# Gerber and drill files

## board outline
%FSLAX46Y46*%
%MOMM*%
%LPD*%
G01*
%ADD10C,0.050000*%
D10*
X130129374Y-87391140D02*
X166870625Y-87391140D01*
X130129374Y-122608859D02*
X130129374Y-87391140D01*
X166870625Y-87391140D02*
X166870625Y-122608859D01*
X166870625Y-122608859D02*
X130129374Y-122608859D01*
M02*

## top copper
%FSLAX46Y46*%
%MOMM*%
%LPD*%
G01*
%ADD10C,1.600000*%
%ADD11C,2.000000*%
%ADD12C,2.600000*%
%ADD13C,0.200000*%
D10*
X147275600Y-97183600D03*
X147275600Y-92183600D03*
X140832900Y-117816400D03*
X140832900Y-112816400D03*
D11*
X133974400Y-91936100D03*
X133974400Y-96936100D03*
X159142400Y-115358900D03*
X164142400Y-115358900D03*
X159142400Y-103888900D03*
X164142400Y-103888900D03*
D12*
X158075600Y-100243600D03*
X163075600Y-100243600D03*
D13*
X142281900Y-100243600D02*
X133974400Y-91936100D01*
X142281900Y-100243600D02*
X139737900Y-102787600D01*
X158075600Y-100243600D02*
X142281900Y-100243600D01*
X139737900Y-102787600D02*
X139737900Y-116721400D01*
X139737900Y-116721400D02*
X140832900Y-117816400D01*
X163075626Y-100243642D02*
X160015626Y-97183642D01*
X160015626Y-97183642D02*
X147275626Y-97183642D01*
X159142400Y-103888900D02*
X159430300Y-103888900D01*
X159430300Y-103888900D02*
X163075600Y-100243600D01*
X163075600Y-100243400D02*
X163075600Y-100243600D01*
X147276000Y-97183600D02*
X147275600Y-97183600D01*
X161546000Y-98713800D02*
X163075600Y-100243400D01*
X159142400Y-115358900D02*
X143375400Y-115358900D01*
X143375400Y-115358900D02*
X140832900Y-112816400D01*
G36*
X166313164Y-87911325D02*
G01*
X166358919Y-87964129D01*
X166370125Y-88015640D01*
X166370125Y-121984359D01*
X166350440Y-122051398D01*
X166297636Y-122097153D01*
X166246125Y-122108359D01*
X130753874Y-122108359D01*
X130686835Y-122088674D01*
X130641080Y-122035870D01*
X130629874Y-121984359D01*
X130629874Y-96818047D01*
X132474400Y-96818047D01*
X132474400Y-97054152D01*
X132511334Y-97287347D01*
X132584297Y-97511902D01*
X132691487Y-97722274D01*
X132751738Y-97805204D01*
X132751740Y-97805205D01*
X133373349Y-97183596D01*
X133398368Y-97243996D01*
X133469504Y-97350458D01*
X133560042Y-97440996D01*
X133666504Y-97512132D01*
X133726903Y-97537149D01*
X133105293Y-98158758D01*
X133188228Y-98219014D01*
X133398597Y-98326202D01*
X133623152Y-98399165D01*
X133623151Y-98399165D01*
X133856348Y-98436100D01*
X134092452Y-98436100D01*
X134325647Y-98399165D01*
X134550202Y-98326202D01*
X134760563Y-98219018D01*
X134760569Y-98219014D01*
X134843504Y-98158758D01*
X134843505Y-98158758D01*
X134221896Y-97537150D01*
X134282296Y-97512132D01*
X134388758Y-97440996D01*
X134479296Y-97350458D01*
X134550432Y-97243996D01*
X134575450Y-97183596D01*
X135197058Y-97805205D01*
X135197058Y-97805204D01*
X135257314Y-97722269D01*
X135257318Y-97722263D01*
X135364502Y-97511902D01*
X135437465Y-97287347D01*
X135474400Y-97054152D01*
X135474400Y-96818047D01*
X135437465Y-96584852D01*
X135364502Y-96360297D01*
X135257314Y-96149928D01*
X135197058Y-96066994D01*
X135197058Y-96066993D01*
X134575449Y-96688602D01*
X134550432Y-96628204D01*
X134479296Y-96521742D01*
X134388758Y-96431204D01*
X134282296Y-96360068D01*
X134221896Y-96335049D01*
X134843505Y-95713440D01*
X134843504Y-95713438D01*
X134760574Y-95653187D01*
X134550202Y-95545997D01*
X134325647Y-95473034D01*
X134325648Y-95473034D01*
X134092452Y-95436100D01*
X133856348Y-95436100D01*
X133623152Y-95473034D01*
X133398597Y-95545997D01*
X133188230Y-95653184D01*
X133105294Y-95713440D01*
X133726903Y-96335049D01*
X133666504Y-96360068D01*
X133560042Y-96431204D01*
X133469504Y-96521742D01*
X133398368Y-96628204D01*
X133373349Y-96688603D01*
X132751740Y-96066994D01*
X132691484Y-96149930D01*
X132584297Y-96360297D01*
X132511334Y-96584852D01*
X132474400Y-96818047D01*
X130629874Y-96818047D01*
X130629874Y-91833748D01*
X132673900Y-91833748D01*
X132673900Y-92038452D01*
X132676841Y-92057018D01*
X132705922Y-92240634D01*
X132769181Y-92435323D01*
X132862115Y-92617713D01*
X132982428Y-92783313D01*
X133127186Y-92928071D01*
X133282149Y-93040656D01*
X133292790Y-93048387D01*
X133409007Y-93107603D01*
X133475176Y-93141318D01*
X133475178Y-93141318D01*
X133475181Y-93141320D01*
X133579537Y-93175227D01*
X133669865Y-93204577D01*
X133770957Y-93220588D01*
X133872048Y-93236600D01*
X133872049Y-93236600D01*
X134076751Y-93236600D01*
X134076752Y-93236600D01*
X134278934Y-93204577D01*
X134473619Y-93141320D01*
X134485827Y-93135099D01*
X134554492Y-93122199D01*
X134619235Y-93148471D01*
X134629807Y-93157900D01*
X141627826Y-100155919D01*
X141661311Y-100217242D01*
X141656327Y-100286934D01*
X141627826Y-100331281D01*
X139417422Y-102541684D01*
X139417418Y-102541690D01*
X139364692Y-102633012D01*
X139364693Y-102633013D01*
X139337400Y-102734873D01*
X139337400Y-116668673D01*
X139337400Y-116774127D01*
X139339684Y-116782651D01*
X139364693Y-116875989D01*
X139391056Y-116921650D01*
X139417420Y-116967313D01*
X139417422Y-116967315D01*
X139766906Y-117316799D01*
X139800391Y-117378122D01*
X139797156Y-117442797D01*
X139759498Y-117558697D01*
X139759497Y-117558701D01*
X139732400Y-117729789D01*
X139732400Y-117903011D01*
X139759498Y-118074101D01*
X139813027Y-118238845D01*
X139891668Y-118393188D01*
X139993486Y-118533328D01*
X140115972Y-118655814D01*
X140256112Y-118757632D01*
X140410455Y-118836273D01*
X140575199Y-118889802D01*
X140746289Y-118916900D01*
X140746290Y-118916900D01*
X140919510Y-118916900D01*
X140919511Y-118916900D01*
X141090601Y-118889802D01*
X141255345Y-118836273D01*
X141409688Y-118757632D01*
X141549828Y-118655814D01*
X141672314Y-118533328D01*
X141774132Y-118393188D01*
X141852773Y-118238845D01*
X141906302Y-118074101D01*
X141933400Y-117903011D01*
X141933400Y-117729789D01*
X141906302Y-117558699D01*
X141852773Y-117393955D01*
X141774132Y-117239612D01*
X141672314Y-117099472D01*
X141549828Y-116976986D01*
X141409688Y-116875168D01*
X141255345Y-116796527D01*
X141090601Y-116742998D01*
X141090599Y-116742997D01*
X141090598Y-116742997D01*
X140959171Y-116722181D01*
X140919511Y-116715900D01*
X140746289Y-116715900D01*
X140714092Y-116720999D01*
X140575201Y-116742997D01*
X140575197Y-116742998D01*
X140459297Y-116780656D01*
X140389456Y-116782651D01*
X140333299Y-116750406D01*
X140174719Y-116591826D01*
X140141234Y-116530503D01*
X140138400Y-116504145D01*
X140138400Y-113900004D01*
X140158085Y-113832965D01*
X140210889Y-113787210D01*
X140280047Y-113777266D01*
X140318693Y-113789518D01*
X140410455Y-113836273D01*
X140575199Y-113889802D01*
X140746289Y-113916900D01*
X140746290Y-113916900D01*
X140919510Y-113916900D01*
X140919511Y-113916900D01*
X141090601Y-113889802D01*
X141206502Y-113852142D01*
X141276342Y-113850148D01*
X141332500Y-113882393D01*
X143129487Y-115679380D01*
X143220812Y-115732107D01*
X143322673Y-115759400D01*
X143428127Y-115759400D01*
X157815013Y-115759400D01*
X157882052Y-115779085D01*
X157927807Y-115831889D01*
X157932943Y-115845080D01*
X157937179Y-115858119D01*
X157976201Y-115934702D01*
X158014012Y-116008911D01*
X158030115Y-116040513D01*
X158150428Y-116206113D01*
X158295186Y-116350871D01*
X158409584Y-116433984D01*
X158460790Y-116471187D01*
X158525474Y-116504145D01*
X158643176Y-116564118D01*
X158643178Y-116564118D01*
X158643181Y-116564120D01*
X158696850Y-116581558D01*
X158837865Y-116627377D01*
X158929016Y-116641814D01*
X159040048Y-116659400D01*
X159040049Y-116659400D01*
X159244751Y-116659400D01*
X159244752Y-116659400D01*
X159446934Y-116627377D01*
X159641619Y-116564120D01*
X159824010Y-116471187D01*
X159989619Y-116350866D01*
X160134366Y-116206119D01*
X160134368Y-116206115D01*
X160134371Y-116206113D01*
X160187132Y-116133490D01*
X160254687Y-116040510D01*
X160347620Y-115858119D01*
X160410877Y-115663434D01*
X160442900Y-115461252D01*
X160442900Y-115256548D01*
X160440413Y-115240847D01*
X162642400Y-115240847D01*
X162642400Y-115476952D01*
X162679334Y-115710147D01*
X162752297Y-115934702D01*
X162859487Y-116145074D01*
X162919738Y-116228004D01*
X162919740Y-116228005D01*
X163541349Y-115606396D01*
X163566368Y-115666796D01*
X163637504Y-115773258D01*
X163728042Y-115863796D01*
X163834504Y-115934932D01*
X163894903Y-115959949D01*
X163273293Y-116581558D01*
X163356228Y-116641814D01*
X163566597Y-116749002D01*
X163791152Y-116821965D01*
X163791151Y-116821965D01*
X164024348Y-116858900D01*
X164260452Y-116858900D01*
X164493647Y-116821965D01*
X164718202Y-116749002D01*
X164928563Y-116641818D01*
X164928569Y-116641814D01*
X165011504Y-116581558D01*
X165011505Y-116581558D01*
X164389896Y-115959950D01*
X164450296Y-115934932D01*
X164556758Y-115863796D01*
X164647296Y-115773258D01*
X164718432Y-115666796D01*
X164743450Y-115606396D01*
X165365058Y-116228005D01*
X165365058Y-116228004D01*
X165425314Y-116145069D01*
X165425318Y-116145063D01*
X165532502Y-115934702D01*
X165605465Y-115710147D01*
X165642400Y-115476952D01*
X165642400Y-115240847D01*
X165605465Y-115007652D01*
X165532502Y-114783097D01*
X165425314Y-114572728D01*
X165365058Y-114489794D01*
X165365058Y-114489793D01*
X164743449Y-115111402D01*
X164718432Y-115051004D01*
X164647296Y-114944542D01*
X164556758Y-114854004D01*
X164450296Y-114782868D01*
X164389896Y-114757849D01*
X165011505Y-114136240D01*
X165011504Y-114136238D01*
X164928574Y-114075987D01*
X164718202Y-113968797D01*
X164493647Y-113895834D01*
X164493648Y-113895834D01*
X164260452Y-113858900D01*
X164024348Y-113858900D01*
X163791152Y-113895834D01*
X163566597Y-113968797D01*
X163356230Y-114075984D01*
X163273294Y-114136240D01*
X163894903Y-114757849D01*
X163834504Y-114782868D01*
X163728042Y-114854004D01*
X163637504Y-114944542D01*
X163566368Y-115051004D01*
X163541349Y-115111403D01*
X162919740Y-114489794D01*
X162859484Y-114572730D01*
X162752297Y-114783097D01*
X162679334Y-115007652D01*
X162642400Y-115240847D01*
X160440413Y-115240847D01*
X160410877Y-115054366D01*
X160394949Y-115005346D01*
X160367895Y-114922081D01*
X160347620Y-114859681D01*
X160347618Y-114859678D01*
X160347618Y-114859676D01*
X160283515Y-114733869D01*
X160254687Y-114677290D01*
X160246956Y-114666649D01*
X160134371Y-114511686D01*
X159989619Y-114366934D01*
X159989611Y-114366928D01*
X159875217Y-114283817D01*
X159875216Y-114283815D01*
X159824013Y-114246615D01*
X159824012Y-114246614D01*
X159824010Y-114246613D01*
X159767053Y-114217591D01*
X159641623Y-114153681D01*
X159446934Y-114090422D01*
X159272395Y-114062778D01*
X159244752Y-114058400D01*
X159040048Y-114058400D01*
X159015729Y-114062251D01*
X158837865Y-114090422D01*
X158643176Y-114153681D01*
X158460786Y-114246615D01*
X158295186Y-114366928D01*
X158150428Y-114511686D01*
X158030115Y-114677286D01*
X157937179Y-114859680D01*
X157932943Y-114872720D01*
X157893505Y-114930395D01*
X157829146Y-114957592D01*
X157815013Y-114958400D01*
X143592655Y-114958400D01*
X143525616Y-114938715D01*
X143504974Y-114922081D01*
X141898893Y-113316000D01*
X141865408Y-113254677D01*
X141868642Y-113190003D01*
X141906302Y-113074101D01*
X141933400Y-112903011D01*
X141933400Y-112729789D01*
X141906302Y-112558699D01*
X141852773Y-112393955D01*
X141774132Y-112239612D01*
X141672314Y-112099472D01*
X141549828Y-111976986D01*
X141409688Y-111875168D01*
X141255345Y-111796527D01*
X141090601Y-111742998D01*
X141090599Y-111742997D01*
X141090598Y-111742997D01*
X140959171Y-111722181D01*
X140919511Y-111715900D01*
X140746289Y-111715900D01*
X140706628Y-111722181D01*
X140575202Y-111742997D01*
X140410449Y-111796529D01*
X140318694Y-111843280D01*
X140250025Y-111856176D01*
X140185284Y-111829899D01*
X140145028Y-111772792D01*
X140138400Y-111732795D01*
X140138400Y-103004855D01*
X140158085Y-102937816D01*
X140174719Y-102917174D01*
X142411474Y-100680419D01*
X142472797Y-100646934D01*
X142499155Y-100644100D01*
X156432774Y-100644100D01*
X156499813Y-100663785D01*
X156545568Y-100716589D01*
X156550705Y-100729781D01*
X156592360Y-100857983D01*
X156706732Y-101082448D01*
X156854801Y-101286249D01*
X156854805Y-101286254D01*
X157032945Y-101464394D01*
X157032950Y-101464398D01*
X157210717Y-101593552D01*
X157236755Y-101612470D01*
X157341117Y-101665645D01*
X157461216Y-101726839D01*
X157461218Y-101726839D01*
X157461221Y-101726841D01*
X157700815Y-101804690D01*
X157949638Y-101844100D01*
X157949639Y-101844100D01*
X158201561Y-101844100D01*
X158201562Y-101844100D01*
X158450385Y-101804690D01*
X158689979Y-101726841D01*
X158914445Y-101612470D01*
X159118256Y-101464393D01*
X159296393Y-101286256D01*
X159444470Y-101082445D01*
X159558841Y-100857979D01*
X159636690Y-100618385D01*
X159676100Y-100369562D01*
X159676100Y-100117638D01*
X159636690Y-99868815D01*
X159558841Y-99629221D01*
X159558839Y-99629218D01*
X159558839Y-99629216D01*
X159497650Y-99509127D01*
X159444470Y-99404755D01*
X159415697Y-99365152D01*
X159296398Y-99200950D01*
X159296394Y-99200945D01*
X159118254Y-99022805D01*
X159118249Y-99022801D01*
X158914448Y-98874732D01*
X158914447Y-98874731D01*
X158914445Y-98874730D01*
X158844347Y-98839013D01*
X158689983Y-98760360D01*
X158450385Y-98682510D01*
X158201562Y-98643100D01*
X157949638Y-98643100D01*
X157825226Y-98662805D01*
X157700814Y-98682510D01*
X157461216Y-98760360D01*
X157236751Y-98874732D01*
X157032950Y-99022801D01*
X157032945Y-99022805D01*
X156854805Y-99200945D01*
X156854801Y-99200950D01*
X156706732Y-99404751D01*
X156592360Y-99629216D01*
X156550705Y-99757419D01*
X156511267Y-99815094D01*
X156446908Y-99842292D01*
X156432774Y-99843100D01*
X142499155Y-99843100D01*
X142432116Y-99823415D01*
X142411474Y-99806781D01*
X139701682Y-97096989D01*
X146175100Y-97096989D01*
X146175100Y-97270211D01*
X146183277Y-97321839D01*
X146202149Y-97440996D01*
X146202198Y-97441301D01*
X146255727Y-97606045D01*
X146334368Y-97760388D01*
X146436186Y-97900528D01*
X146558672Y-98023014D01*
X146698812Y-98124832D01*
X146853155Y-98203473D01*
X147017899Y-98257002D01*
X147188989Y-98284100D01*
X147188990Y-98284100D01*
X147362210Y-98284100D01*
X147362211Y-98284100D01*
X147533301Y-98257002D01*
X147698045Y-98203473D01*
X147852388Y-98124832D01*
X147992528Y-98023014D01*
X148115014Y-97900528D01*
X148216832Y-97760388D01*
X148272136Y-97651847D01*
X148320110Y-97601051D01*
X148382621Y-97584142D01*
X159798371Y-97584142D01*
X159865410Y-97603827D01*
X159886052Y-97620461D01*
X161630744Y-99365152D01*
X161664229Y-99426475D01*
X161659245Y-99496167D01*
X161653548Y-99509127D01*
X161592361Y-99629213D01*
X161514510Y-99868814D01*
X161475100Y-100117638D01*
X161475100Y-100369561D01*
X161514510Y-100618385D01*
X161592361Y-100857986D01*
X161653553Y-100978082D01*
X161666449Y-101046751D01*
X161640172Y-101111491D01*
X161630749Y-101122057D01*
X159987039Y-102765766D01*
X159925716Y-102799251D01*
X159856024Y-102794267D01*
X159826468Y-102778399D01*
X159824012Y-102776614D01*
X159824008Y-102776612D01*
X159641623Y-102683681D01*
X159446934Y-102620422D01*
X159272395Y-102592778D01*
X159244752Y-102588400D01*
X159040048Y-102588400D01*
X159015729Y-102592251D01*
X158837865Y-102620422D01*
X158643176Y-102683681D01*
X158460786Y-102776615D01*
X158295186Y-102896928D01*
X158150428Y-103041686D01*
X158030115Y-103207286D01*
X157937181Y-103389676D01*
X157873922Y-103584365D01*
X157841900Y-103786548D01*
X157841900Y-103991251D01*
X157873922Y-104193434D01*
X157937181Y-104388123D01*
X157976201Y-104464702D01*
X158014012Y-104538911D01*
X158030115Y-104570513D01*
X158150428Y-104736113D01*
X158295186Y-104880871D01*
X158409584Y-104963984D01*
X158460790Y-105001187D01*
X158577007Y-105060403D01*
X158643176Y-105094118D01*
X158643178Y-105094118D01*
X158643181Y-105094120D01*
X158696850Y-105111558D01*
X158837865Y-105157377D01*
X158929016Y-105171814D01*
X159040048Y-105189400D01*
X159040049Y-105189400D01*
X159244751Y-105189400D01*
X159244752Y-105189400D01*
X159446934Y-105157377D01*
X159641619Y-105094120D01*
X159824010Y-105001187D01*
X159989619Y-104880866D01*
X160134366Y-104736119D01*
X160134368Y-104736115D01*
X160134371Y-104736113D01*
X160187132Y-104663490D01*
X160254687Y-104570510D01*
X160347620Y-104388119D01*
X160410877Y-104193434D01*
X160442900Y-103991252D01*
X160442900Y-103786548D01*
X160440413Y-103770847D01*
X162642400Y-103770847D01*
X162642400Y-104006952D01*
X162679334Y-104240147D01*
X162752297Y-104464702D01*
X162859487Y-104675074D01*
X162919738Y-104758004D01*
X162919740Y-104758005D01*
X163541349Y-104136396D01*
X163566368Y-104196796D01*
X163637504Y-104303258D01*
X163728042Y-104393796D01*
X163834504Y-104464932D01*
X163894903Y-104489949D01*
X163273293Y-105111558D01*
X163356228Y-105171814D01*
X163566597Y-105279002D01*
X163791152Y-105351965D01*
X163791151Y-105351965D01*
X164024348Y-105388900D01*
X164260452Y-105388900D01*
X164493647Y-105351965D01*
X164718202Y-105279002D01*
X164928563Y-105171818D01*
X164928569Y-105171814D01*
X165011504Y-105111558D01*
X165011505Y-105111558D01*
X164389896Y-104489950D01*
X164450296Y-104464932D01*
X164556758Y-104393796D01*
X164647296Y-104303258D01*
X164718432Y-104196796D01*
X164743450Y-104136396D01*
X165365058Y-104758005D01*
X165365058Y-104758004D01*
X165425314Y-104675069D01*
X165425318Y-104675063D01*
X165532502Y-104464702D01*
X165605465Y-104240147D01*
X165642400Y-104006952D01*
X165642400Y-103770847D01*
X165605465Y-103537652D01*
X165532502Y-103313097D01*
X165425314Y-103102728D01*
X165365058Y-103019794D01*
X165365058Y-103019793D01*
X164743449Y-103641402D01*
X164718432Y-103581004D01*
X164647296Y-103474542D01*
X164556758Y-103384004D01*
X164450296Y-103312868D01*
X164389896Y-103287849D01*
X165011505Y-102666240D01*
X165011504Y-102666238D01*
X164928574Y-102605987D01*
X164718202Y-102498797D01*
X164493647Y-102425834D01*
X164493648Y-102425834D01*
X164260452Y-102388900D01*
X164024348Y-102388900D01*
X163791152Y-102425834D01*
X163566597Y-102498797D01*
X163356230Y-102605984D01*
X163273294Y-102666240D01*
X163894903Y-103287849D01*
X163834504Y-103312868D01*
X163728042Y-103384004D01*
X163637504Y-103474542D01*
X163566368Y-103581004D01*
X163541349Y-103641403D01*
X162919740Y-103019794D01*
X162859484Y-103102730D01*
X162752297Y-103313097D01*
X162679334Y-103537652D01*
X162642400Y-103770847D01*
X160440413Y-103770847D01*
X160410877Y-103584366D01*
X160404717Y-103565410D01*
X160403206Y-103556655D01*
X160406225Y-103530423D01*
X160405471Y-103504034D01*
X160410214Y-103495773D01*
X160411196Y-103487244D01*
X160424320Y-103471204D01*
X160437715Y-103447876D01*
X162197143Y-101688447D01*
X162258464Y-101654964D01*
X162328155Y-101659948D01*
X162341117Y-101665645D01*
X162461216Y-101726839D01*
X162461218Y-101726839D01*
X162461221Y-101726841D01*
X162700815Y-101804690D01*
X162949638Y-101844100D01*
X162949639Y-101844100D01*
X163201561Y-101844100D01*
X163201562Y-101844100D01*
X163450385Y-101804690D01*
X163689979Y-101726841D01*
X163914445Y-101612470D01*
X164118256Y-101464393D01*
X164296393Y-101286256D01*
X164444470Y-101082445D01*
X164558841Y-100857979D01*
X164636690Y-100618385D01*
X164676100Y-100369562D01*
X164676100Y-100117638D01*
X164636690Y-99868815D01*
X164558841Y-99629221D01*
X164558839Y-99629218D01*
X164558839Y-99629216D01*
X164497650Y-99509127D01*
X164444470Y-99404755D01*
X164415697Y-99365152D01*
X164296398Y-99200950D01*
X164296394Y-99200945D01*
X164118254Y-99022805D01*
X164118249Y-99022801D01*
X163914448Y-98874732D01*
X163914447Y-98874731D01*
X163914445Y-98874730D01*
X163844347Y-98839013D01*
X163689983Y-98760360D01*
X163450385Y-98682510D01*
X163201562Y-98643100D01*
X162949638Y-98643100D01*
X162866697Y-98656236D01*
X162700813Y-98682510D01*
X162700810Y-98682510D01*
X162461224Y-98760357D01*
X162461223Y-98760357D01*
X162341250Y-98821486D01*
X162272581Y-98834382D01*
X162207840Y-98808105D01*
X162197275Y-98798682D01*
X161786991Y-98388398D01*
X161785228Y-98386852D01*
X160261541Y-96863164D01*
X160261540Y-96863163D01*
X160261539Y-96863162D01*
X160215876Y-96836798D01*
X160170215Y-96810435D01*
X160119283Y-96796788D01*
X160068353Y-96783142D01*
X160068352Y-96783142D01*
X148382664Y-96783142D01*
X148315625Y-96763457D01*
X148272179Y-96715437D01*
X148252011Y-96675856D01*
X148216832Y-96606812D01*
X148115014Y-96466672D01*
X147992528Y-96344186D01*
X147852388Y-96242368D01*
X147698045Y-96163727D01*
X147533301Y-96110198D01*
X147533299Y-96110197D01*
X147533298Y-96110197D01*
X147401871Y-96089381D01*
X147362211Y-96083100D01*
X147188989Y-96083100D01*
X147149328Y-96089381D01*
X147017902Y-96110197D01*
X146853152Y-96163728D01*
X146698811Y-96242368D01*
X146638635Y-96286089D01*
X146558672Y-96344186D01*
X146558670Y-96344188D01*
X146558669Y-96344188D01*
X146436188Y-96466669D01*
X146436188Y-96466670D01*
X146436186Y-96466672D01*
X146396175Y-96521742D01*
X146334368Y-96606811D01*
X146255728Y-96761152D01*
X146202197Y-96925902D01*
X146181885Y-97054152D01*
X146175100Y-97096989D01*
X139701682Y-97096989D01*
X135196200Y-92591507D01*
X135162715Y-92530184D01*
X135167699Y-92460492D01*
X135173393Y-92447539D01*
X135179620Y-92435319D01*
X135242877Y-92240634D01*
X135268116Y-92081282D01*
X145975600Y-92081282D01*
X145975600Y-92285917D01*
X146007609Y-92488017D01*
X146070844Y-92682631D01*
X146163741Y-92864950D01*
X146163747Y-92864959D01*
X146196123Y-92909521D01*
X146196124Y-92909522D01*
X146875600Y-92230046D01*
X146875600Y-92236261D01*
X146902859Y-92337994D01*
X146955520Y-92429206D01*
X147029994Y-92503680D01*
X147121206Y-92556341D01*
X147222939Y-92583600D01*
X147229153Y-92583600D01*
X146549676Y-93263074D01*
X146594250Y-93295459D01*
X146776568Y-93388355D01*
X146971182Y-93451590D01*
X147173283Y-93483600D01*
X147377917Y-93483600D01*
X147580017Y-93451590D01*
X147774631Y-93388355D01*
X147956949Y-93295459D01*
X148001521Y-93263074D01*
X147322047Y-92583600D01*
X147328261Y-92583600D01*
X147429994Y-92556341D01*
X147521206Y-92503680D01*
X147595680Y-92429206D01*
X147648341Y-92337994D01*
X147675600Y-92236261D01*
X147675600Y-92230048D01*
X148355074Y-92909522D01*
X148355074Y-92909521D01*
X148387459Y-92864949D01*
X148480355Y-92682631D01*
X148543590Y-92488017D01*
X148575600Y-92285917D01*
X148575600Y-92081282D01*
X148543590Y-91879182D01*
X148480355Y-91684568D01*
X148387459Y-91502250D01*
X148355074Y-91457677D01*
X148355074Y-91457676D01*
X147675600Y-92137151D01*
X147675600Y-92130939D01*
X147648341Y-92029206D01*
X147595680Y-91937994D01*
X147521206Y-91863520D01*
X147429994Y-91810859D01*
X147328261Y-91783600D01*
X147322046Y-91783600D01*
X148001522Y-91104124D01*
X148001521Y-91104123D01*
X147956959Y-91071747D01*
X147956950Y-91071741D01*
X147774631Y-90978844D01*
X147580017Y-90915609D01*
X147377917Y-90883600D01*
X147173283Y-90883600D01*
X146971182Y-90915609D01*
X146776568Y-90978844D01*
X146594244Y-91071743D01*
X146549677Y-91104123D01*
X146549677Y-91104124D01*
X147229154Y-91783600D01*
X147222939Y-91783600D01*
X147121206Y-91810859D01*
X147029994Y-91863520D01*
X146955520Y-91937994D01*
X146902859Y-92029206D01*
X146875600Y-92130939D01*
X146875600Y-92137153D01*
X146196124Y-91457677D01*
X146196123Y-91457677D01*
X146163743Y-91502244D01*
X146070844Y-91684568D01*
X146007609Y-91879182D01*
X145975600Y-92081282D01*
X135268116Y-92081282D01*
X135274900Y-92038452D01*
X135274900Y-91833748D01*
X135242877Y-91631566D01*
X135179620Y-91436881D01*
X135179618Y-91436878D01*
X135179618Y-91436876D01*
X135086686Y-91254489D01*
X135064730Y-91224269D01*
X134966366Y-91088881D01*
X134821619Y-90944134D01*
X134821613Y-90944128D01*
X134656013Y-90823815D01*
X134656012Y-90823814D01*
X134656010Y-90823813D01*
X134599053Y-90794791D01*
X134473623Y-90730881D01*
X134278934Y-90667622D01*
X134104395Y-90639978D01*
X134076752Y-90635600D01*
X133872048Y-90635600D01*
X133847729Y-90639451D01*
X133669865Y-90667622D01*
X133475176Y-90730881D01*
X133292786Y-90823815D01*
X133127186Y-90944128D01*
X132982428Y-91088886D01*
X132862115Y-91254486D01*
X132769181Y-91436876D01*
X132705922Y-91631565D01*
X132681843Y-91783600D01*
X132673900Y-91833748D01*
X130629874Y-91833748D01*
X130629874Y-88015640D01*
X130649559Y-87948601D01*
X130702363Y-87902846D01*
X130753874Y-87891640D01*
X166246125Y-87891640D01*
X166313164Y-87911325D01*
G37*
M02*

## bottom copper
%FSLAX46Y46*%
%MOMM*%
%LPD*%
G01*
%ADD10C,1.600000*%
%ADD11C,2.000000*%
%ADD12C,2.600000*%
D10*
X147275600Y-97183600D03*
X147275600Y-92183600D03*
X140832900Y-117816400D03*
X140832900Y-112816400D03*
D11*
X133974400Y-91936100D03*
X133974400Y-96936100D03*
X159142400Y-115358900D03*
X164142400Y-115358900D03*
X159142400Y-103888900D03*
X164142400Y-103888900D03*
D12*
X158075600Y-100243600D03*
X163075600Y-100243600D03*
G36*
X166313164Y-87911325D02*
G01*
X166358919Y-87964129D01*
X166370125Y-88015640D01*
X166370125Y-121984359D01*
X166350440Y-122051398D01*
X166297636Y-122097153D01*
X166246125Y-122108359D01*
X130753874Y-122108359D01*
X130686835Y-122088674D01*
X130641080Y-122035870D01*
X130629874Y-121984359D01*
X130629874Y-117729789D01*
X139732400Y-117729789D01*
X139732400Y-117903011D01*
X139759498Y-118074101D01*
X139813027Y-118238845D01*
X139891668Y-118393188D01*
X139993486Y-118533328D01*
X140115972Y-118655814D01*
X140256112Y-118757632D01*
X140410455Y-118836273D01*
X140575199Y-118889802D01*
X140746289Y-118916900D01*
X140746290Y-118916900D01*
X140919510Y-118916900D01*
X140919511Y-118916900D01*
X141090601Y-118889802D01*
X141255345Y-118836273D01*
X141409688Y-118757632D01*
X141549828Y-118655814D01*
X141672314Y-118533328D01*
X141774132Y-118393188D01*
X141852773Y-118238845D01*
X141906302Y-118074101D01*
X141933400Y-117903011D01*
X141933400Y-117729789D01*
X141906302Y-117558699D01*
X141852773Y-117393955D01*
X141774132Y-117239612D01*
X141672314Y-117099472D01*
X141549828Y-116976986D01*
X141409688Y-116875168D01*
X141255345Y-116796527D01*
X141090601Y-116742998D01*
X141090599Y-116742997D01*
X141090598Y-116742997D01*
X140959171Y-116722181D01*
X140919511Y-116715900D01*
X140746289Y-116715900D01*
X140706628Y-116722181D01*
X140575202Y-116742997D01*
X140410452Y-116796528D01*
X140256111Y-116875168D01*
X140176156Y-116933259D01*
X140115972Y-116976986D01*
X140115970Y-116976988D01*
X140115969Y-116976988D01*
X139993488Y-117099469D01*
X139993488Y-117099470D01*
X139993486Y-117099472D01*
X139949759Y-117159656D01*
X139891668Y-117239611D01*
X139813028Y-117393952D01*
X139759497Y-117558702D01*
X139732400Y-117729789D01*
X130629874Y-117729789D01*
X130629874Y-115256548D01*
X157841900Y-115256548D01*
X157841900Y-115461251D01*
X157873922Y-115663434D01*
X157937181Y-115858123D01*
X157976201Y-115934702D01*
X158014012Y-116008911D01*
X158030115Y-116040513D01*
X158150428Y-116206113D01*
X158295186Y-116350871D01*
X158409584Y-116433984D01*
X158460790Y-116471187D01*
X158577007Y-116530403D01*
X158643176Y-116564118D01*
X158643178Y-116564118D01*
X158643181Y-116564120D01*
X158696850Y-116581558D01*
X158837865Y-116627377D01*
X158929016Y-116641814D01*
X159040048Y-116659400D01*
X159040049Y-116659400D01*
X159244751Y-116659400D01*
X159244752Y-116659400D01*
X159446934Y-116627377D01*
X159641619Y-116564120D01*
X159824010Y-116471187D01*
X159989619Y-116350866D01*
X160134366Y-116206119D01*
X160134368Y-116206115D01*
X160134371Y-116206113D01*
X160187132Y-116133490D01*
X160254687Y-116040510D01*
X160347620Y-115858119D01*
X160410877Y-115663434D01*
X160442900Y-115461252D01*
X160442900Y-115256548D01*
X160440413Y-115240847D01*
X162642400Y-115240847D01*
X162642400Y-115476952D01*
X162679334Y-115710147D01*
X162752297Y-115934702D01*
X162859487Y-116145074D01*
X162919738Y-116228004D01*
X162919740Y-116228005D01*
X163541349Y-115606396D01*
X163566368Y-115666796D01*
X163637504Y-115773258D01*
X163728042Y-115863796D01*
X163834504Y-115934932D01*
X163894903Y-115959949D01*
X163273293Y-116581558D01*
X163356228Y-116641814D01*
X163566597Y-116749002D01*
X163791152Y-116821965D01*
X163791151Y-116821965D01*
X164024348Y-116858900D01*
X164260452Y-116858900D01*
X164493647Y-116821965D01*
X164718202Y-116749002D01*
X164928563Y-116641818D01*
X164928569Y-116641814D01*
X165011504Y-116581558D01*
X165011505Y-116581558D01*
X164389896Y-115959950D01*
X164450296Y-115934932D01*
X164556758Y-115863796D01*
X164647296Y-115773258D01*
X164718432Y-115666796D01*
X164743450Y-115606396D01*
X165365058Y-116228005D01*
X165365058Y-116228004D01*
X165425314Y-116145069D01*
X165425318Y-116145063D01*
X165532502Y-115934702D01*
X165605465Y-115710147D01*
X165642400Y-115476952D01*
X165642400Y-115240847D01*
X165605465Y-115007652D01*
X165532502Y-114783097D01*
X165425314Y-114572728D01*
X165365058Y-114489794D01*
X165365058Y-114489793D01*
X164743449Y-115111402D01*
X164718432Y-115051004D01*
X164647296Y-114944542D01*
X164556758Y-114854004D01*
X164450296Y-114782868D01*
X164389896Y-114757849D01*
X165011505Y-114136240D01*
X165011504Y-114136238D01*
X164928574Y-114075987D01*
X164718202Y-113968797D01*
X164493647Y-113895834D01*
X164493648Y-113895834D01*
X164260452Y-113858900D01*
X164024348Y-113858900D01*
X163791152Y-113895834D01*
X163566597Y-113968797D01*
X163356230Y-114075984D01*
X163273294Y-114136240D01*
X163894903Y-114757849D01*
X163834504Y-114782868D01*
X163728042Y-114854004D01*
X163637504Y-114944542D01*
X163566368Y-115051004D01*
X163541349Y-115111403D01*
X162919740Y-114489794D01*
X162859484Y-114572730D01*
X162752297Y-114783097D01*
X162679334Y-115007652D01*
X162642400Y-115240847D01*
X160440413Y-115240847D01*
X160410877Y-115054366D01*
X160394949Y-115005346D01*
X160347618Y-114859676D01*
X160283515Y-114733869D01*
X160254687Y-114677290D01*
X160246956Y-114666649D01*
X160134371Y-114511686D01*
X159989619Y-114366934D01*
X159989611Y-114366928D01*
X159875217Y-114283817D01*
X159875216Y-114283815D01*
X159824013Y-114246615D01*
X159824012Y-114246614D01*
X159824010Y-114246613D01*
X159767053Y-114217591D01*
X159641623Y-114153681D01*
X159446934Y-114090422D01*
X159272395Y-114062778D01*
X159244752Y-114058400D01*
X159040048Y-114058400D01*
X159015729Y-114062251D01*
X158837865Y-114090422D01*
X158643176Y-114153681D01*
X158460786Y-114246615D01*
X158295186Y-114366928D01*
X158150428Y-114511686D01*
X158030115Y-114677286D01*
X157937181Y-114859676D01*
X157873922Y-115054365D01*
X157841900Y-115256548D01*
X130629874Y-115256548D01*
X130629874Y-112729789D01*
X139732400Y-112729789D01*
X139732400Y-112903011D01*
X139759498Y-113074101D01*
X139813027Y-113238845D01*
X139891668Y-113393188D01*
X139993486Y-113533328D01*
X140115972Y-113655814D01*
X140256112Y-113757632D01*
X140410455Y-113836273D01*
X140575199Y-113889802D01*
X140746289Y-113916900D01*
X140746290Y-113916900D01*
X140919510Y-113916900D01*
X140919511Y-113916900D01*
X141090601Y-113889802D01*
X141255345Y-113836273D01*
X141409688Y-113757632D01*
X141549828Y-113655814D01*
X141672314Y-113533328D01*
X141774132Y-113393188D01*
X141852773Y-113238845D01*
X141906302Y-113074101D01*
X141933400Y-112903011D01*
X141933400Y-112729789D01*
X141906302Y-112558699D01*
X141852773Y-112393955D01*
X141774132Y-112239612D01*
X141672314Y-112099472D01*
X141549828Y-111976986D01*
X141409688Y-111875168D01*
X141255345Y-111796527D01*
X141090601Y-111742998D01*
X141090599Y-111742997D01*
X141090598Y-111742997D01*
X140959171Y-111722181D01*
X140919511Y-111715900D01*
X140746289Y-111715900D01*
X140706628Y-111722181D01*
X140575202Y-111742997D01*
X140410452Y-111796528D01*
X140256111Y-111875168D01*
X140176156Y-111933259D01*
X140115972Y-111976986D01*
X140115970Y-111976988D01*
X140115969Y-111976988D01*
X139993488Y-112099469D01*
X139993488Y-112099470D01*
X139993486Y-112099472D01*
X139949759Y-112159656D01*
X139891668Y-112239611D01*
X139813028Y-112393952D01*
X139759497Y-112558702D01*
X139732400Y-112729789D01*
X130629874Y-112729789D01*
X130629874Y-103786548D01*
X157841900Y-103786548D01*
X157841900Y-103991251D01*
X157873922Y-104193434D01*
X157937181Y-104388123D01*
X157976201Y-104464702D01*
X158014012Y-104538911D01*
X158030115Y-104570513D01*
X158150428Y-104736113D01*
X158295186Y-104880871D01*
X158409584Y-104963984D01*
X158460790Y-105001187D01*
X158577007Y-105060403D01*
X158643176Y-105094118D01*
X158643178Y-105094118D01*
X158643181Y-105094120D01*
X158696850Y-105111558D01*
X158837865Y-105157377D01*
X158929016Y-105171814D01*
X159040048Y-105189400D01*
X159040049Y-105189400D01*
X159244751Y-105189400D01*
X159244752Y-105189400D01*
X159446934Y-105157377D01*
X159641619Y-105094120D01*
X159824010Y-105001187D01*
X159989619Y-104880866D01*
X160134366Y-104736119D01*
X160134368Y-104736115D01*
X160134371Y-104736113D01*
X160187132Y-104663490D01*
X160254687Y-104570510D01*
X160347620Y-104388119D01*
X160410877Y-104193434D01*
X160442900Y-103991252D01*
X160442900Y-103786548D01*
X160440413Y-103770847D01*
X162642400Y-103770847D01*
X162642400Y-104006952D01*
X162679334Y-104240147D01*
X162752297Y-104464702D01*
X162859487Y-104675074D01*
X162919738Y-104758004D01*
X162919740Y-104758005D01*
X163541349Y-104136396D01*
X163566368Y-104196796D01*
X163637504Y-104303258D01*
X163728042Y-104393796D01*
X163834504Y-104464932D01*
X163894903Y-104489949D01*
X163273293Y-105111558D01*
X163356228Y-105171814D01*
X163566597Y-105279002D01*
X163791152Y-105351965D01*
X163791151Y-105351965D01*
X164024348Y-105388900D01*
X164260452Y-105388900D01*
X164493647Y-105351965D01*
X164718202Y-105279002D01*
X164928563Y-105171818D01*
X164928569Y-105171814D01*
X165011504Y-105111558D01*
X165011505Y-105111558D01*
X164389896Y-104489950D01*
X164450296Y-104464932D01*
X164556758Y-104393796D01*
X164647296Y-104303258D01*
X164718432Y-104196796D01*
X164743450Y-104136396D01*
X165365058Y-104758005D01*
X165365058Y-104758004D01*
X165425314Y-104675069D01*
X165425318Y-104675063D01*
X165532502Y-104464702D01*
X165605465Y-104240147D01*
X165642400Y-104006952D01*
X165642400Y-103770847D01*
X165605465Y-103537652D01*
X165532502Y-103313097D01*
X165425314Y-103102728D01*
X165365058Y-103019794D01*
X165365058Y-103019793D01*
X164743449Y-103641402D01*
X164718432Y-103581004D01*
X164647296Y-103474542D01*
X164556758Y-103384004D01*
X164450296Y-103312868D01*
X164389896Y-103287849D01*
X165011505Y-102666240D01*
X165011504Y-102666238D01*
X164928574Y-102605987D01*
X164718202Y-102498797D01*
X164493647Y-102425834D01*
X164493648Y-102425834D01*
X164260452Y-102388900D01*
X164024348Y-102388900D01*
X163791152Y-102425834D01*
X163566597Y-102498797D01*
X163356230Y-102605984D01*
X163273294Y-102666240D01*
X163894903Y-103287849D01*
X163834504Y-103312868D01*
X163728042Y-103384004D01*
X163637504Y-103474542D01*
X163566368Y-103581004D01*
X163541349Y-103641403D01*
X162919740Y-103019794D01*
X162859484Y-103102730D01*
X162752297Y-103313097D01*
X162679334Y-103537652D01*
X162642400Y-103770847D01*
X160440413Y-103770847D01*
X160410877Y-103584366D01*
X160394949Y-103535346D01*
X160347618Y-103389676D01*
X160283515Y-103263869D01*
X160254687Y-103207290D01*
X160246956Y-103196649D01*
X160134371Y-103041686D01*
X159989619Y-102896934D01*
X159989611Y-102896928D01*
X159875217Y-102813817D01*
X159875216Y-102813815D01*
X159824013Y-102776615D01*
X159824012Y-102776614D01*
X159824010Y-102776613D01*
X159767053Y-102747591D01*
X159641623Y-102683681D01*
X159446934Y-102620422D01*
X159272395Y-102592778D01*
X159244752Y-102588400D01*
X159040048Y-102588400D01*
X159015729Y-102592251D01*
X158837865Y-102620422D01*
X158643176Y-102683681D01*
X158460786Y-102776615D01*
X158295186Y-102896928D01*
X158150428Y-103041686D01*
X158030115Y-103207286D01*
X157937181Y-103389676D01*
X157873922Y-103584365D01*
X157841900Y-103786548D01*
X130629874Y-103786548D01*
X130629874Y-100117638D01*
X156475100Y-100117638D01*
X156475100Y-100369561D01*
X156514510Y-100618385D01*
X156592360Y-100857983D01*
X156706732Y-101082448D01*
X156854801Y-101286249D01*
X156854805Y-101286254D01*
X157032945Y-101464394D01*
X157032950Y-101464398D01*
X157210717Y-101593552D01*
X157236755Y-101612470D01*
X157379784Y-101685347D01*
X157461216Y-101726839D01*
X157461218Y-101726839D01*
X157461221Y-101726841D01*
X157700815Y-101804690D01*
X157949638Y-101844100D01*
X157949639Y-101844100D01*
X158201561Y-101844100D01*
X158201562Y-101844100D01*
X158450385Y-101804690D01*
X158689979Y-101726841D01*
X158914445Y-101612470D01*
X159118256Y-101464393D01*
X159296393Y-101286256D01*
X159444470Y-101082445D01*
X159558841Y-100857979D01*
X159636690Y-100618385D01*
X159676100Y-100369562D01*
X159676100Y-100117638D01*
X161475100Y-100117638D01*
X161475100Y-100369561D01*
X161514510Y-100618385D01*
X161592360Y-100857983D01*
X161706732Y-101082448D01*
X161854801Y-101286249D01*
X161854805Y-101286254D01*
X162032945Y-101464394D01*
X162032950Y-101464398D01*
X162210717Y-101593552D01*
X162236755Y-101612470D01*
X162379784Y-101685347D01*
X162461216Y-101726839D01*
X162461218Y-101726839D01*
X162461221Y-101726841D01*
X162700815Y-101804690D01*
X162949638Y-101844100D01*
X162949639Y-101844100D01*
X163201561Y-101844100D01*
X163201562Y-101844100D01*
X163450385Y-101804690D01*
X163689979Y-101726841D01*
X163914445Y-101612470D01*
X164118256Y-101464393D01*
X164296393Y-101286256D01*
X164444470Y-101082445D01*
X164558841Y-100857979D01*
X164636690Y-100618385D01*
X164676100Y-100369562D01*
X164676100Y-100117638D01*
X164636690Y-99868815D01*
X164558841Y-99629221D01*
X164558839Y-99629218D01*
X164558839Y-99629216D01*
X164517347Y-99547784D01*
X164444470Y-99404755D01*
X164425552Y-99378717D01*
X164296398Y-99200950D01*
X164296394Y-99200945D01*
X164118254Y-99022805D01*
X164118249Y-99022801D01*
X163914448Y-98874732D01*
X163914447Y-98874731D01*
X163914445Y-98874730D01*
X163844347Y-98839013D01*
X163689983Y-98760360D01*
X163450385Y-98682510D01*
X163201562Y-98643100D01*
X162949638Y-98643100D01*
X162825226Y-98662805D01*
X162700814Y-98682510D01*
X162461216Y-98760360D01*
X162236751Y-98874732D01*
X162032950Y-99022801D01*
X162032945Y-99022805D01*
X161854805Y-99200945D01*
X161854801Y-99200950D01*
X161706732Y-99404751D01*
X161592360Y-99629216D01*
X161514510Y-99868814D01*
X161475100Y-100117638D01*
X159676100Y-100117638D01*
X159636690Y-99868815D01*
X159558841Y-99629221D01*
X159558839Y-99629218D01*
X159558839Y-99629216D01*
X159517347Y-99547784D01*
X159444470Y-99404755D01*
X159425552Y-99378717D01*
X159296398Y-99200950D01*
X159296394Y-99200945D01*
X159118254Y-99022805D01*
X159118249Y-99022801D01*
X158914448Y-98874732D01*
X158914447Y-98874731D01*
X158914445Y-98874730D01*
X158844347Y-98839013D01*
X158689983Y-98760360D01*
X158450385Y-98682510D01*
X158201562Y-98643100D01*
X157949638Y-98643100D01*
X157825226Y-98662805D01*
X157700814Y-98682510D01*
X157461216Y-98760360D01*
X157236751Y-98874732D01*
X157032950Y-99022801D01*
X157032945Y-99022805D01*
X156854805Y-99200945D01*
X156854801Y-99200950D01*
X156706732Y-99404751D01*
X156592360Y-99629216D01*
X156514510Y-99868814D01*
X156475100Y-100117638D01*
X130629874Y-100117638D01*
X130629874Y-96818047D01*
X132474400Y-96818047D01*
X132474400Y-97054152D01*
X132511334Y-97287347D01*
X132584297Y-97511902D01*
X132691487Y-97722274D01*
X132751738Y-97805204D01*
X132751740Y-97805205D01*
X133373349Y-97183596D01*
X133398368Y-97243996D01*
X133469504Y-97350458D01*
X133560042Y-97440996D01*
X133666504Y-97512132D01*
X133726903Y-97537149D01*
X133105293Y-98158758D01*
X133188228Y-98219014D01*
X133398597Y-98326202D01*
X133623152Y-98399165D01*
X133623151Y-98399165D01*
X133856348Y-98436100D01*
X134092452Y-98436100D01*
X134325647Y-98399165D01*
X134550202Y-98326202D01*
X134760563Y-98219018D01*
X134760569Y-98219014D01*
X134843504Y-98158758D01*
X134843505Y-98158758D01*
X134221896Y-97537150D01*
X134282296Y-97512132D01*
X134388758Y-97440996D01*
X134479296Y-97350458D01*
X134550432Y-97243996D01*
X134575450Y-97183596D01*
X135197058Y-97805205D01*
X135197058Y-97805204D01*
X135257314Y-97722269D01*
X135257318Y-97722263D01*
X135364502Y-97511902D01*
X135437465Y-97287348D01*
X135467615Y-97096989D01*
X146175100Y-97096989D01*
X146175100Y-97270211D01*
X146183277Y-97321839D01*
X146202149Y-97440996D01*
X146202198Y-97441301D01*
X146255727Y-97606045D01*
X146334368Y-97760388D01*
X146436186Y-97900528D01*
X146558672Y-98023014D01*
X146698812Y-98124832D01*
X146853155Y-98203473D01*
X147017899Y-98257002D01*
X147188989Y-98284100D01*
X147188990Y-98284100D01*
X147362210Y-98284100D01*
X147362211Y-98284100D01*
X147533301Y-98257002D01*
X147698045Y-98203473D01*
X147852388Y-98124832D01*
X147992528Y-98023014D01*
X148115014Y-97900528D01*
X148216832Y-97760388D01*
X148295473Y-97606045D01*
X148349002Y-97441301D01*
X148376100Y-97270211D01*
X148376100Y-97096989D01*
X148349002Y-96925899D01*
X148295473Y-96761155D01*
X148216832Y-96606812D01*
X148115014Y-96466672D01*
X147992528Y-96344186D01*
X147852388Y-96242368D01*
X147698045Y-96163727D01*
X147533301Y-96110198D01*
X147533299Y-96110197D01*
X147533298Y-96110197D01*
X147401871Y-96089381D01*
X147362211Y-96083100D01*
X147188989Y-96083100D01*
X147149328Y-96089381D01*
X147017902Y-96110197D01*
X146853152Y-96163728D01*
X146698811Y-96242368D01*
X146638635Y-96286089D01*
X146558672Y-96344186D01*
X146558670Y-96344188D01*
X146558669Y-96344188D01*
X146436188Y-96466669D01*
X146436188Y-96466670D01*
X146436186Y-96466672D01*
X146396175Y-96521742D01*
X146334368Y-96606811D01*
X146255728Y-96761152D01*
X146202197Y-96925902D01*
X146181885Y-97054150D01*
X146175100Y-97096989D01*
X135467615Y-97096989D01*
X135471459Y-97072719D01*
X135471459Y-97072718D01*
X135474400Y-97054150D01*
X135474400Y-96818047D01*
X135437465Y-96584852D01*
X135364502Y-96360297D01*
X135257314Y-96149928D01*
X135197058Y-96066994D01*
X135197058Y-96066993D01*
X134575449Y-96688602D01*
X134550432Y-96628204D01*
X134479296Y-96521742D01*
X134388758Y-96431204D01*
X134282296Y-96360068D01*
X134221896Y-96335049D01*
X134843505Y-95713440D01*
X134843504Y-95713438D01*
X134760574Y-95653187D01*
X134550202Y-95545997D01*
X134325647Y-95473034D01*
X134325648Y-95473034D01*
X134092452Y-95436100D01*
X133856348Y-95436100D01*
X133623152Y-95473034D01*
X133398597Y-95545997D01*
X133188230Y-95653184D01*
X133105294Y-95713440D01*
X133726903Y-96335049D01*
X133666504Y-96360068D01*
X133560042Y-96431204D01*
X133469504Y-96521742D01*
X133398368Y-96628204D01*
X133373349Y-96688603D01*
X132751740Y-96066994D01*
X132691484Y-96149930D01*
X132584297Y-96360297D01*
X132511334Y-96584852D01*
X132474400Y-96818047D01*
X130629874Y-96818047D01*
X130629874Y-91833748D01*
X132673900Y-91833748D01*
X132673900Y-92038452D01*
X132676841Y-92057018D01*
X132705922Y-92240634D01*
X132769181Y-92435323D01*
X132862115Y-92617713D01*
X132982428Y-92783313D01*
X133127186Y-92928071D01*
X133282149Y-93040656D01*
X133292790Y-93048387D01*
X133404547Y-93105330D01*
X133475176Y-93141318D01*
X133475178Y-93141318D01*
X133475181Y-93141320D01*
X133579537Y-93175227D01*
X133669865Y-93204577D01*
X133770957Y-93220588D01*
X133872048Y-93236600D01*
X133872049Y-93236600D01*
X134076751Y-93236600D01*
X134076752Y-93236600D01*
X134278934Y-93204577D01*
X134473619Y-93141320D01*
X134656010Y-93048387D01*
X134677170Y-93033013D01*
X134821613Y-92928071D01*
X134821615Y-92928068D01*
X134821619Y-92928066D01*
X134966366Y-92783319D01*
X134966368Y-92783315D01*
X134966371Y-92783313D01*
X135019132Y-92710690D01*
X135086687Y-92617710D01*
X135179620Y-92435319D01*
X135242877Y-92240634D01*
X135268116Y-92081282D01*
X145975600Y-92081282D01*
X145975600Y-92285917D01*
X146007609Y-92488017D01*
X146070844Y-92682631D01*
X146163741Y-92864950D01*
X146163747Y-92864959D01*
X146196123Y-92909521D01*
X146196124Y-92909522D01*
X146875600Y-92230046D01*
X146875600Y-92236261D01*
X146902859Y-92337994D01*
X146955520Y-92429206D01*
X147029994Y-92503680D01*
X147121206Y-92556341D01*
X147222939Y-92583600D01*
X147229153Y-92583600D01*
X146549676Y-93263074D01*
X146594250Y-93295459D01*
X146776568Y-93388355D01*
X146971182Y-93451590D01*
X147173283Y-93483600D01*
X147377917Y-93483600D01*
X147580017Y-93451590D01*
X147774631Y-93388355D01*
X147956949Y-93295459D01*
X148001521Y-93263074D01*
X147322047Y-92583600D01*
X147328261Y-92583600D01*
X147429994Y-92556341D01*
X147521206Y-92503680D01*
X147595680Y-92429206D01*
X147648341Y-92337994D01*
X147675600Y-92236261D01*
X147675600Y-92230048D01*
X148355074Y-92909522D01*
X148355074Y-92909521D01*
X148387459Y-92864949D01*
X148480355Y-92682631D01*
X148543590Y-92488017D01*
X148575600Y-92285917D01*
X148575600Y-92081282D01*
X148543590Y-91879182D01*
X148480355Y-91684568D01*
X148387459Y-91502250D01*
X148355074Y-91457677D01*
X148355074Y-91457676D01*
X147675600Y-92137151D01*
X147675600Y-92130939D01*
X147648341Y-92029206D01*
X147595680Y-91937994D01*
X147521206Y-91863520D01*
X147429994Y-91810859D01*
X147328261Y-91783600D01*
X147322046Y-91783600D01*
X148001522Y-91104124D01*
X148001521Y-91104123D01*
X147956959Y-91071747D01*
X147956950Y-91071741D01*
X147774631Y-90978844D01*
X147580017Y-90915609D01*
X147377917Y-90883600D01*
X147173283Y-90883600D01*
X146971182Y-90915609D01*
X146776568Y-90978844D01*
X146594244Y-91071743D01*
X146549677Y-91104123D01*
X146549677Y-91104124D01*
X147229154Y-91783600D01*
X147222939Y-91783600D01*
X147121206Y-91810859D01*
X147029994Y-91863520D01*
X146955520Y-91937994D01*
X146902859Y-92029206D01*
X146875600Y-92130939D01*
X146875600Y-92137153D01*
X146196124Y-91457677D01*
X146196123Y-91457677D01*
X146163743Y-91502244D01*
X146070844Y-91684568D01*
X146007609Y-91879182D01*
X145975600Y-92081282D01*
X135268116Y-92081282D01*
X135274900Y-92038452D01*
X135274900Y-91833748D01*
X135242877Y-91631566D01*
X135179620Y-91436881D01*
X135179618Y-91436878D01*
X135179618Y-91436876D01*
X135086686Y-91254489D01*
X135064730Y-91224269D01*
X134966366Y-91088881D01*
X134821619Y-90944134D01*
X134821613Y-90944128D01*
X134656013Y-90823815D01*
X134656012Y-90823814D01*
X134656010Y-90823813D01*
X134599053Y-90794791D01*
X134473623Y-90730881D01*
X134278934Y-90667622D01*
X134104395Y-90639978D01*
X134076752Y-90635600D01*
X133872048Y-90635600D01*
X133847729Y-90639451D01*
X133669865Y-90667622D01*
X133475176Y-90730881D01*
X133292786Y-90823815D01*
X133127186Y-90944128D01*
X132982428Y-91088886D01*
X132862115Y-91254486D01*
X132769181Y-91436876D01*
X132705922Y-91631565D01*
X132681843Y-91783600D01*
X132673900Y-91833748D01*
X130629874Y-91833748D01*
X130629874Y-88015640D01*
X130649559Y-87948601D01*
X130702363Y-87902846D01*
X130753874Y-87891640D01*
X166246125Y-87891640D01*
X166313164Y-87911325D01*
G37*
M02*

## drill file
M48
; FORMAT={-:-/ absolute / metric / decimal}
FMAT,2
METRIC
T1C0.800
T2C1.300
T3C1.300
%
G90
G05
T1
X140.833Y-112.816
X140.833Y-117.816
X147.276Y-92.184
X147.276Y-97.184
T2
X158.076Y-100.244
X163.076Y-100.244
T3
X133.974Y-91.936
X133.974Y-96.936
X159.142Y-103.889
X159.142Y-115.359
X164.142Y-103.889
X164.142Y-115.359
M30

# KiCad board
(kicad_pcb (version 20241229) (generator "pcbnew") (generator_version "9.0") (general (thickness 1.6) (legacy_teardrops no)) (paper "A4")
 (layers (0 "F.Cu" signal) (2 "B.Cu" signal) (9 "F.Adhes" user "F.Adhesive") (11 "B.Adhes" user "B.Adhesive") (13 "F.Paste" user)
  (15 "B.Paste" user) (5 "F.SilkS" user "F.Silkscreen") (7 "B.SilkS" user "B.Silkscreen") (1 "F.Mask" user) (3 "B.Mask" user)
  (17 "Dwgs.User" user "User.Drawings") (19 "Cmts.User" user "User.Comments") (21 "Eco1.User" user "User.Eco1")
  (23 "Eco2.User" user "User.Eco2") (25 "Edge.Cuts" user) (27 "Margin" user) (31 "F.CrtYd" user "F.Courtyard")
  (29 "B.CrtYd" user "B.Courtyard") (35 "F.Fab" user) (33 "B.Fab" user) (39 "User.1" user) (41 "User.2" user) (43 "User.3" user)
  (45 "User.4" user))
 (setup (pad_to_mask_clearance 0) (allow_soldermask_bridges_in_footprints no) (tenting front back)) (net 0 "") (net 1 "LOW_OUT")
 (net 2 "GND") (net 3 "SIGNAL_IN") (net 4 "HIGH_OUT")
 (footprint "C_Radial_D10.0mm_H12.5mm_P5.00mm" (layer "F.Cu") (at 147.2756 97.1836 90)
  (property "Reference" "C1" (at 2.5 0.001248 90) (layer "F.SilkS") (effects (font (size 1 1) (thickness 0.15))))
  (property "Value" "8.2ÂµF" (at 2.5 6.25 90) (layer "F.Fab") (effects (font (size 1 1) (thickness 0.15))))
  (pad "1" thru_hole circle (at 0 0 90) (size 1.6 1.6) (drill 0.8) (layers "*.Cu" "*.Mask") (remove_unused_layers no) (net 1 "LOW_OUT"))
  (pad "2" thru_hole circle (at 5 0 90) (size 1.6 1.6) (drill 0.8) (layers "*.Cu" "*.Mask") (remove_unused_layers no) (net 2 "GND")))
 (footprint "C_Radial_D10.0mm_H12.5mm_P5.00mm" (layer "F.Cu") (at 140.8329 117.8164 90)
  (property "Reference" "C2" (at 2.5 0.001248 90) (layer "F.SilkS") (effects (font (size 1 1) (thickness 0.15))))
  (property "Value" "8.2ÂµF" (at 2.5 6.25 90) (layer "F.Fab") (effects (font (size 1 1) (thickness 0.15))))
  (pad "1" thru_hole circle (at 0 0 90) (size 1.6 1.6) (drill 0.8) (layers "*.Cu" "*.Mask") (remove_unused_layers no) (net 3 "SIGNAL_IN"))
  (pad "2" thru_hole circle (at 5 0 90) (size 1.6 1.6) (drill 0.8) (layers "*.Cu" "*.Mask") (remove_unused_layers no) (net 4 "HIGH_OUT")))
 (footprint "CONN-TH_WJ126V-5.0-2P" (layer "F.Cu") (at 133.9744 94.4361)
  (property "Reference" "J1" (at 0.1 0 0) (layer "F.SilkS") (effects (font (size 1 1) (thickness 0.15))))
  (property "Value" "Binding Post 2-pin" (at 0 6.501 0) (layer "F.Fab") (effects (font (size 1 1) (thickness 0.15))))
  (pad "1" thru_hole circle (at 0 -2.5) (size 2 2) (drill 1.300022) (layers "*.Cu" "*.Mask") (remove_unused_layers no) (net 3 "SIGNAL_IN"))
  (pad "2" thru_hole circle (at 0 2.5) (size 2 2) (drill 1.300022) (layers "*.Cu" "*.Mask") (remove_unused_layers no) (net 2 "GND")))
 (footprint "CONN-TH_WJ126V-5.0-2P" (layer "F.Cu") (at 161.6424 115.3589 90)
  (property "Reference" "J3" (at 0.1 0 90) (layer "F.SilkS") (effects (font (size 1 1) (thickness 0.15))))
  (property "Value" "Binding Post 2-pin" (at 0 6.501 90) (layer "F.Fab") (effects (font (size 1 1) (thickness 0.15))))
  (pad "1" thru_hole circle (at 0 -2.5 90) (size 2 2) (drill 1.300022) (layers "*.Cu" "*.Mask") (remove_unused_layers no) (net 4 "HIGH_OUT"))
  (pad "2" thru_hole circle (at 0 2.5 90) (size 2 2) (drill 1.300022) (layers "*.Cu" "*.Mask") (remove_unused_layers no) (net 2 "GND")))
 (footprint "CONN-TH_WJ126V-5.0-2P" (layer "F.Cu") (at 161.6424 103.8889 90)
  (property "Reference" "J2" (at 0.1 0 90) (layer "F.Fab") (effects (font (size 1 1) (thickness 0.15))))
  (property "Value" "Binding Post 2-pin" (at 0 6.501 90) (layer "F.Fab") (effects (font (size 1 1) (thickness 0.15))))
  (pad "1" thru_hole circle (at 0 -2.5 90) (size 2 2) (drill 1.300022) (layers "*.Cu" "*.Mask") (remove_unused_layers no) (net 1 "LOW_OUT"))
  (pad "2" thru_hole circle (at 0 2.5 90) (size 2 2) (drill 1.300022) (layers "*.Cu" "*.Mask") (remove_unused_layers no) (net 2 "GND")))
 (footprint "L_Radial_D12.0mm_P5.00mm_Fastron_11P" (layer "B.Cu") (at 158.0756 100.2436)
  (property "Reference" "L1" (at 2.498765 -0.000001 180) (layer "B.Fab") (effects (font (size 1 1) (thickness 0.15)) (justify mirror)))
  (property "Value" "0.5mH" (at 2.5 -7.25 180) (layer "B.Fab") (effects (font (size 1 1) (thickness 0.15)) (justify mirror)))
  (pad "1" thru_hole circle (at 0 0) (size 2.6 2.6) (drill 1.3) (layers "*.Cu" "*.Mask") (remove_unused_layers no) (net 3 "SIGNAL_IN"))
  (pad "2" thru_hole circle (at 5 0) (size 2.6 2.6) (drill 1.3) (layers "*.Cu" "*.Mask") (remove_unused_layers no) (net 1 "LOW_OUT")))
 (gr_line (start 130.129374 87.39114) (end 166.870625 87.39114) (stroke (width 0.05) (type default)) (layer "Edge.Cuts"))
 (gr_line (start 130.129374 122.608859) (end 130.129374 87.39114) (stroke (width 0.05) (type default)) (layer "Edge.Cuts"))
 (gr_line (start 166.870625 87.39114) (end 166.870625 122.608859) (stroke (width 0.05) (type default)) (layer "Edge.Cuts"))
 (gr_line (start 166.870625 122.608859) (end 130.129374 122.608859) (stroke (width 0.05) (type default)) (layer "Edge.Cuts"))
 (segment (start 142.2819 100.2436) (end 133.9744 91.9361) (width 0.2) (layer "F.Cu") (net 3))
 (segment (start 142.2819 100.2436) (end 139.7379 102.7876) (width 0.2) (layer "F.Cu") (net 3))
 (segment (start 158.0756 100.2436) (end 142.2819 100.2436) (width 0.2) (layer "F.Cu") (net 3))
 (segment (start 139.7379 102.7876) (end 139.7379 116.7214) (width 0.2) (layer "F.Cu") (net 3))
 (segment (start 139.7379 116.7214) (end 140.8329 117.8164) (width 0.2) (layer "F.Cu") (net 3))
 (segment (start 163.075626 100.243642) (end 160.015626 97.183642) (width 0.2) (layer "F.Cu") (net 1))
 (segment (start 160.015626 97.183642) (end 147.275626 97.183642) (width 0.2) (layer "F.Cu") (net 1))
 (segment (start 159.1424 103.8889) (end 159.4303 103.8889) (width 0.2) (layer "F.Cu") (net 1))
 (segment (start 159.4303 103.8889) (end 163.0756 100.2436) (width 0.2) (layer "F.Cu") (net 1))
 (segment (start 163.0756 100.2434) (end 163.0756 100.2436) (width 0.2) (layer "F.Cu") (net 1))
 (segment (start 147.276 97.1836) (end 147.2756 97.1836) (width 0.2) (layer "F.Cu") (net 1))
 (segment (start 161.546 98.7138) (end 163.0756 100.2434) (width 0.2) (layer "F.Cu") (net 1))
 (segment (start 159.1424 115.3589) (end 143.3754 115.3589) (width 0.2) (layer "F.Cu") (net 4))
 (segment (start 143.3754 115.3589) (end 140.8329 112.8164) (width 0.2) (layer "F.Cu") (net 4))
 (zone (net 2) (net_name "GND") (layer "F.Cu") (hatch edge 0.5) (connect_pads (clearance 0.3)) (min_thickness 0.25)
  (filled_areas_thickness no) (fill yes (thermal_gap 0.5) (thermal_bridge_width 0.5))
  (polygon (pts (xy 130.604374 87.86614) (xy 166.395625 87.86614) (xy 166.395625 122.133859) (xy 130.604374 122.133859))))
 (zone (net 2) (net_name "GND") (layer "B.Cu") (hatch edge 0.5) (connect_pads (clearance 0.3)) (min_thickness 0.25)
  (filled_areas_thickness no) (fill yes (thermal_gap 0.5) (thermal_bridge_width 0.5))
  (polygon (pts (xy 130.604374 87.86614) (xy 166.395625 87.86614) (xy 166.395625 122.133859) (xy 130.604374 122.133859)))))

